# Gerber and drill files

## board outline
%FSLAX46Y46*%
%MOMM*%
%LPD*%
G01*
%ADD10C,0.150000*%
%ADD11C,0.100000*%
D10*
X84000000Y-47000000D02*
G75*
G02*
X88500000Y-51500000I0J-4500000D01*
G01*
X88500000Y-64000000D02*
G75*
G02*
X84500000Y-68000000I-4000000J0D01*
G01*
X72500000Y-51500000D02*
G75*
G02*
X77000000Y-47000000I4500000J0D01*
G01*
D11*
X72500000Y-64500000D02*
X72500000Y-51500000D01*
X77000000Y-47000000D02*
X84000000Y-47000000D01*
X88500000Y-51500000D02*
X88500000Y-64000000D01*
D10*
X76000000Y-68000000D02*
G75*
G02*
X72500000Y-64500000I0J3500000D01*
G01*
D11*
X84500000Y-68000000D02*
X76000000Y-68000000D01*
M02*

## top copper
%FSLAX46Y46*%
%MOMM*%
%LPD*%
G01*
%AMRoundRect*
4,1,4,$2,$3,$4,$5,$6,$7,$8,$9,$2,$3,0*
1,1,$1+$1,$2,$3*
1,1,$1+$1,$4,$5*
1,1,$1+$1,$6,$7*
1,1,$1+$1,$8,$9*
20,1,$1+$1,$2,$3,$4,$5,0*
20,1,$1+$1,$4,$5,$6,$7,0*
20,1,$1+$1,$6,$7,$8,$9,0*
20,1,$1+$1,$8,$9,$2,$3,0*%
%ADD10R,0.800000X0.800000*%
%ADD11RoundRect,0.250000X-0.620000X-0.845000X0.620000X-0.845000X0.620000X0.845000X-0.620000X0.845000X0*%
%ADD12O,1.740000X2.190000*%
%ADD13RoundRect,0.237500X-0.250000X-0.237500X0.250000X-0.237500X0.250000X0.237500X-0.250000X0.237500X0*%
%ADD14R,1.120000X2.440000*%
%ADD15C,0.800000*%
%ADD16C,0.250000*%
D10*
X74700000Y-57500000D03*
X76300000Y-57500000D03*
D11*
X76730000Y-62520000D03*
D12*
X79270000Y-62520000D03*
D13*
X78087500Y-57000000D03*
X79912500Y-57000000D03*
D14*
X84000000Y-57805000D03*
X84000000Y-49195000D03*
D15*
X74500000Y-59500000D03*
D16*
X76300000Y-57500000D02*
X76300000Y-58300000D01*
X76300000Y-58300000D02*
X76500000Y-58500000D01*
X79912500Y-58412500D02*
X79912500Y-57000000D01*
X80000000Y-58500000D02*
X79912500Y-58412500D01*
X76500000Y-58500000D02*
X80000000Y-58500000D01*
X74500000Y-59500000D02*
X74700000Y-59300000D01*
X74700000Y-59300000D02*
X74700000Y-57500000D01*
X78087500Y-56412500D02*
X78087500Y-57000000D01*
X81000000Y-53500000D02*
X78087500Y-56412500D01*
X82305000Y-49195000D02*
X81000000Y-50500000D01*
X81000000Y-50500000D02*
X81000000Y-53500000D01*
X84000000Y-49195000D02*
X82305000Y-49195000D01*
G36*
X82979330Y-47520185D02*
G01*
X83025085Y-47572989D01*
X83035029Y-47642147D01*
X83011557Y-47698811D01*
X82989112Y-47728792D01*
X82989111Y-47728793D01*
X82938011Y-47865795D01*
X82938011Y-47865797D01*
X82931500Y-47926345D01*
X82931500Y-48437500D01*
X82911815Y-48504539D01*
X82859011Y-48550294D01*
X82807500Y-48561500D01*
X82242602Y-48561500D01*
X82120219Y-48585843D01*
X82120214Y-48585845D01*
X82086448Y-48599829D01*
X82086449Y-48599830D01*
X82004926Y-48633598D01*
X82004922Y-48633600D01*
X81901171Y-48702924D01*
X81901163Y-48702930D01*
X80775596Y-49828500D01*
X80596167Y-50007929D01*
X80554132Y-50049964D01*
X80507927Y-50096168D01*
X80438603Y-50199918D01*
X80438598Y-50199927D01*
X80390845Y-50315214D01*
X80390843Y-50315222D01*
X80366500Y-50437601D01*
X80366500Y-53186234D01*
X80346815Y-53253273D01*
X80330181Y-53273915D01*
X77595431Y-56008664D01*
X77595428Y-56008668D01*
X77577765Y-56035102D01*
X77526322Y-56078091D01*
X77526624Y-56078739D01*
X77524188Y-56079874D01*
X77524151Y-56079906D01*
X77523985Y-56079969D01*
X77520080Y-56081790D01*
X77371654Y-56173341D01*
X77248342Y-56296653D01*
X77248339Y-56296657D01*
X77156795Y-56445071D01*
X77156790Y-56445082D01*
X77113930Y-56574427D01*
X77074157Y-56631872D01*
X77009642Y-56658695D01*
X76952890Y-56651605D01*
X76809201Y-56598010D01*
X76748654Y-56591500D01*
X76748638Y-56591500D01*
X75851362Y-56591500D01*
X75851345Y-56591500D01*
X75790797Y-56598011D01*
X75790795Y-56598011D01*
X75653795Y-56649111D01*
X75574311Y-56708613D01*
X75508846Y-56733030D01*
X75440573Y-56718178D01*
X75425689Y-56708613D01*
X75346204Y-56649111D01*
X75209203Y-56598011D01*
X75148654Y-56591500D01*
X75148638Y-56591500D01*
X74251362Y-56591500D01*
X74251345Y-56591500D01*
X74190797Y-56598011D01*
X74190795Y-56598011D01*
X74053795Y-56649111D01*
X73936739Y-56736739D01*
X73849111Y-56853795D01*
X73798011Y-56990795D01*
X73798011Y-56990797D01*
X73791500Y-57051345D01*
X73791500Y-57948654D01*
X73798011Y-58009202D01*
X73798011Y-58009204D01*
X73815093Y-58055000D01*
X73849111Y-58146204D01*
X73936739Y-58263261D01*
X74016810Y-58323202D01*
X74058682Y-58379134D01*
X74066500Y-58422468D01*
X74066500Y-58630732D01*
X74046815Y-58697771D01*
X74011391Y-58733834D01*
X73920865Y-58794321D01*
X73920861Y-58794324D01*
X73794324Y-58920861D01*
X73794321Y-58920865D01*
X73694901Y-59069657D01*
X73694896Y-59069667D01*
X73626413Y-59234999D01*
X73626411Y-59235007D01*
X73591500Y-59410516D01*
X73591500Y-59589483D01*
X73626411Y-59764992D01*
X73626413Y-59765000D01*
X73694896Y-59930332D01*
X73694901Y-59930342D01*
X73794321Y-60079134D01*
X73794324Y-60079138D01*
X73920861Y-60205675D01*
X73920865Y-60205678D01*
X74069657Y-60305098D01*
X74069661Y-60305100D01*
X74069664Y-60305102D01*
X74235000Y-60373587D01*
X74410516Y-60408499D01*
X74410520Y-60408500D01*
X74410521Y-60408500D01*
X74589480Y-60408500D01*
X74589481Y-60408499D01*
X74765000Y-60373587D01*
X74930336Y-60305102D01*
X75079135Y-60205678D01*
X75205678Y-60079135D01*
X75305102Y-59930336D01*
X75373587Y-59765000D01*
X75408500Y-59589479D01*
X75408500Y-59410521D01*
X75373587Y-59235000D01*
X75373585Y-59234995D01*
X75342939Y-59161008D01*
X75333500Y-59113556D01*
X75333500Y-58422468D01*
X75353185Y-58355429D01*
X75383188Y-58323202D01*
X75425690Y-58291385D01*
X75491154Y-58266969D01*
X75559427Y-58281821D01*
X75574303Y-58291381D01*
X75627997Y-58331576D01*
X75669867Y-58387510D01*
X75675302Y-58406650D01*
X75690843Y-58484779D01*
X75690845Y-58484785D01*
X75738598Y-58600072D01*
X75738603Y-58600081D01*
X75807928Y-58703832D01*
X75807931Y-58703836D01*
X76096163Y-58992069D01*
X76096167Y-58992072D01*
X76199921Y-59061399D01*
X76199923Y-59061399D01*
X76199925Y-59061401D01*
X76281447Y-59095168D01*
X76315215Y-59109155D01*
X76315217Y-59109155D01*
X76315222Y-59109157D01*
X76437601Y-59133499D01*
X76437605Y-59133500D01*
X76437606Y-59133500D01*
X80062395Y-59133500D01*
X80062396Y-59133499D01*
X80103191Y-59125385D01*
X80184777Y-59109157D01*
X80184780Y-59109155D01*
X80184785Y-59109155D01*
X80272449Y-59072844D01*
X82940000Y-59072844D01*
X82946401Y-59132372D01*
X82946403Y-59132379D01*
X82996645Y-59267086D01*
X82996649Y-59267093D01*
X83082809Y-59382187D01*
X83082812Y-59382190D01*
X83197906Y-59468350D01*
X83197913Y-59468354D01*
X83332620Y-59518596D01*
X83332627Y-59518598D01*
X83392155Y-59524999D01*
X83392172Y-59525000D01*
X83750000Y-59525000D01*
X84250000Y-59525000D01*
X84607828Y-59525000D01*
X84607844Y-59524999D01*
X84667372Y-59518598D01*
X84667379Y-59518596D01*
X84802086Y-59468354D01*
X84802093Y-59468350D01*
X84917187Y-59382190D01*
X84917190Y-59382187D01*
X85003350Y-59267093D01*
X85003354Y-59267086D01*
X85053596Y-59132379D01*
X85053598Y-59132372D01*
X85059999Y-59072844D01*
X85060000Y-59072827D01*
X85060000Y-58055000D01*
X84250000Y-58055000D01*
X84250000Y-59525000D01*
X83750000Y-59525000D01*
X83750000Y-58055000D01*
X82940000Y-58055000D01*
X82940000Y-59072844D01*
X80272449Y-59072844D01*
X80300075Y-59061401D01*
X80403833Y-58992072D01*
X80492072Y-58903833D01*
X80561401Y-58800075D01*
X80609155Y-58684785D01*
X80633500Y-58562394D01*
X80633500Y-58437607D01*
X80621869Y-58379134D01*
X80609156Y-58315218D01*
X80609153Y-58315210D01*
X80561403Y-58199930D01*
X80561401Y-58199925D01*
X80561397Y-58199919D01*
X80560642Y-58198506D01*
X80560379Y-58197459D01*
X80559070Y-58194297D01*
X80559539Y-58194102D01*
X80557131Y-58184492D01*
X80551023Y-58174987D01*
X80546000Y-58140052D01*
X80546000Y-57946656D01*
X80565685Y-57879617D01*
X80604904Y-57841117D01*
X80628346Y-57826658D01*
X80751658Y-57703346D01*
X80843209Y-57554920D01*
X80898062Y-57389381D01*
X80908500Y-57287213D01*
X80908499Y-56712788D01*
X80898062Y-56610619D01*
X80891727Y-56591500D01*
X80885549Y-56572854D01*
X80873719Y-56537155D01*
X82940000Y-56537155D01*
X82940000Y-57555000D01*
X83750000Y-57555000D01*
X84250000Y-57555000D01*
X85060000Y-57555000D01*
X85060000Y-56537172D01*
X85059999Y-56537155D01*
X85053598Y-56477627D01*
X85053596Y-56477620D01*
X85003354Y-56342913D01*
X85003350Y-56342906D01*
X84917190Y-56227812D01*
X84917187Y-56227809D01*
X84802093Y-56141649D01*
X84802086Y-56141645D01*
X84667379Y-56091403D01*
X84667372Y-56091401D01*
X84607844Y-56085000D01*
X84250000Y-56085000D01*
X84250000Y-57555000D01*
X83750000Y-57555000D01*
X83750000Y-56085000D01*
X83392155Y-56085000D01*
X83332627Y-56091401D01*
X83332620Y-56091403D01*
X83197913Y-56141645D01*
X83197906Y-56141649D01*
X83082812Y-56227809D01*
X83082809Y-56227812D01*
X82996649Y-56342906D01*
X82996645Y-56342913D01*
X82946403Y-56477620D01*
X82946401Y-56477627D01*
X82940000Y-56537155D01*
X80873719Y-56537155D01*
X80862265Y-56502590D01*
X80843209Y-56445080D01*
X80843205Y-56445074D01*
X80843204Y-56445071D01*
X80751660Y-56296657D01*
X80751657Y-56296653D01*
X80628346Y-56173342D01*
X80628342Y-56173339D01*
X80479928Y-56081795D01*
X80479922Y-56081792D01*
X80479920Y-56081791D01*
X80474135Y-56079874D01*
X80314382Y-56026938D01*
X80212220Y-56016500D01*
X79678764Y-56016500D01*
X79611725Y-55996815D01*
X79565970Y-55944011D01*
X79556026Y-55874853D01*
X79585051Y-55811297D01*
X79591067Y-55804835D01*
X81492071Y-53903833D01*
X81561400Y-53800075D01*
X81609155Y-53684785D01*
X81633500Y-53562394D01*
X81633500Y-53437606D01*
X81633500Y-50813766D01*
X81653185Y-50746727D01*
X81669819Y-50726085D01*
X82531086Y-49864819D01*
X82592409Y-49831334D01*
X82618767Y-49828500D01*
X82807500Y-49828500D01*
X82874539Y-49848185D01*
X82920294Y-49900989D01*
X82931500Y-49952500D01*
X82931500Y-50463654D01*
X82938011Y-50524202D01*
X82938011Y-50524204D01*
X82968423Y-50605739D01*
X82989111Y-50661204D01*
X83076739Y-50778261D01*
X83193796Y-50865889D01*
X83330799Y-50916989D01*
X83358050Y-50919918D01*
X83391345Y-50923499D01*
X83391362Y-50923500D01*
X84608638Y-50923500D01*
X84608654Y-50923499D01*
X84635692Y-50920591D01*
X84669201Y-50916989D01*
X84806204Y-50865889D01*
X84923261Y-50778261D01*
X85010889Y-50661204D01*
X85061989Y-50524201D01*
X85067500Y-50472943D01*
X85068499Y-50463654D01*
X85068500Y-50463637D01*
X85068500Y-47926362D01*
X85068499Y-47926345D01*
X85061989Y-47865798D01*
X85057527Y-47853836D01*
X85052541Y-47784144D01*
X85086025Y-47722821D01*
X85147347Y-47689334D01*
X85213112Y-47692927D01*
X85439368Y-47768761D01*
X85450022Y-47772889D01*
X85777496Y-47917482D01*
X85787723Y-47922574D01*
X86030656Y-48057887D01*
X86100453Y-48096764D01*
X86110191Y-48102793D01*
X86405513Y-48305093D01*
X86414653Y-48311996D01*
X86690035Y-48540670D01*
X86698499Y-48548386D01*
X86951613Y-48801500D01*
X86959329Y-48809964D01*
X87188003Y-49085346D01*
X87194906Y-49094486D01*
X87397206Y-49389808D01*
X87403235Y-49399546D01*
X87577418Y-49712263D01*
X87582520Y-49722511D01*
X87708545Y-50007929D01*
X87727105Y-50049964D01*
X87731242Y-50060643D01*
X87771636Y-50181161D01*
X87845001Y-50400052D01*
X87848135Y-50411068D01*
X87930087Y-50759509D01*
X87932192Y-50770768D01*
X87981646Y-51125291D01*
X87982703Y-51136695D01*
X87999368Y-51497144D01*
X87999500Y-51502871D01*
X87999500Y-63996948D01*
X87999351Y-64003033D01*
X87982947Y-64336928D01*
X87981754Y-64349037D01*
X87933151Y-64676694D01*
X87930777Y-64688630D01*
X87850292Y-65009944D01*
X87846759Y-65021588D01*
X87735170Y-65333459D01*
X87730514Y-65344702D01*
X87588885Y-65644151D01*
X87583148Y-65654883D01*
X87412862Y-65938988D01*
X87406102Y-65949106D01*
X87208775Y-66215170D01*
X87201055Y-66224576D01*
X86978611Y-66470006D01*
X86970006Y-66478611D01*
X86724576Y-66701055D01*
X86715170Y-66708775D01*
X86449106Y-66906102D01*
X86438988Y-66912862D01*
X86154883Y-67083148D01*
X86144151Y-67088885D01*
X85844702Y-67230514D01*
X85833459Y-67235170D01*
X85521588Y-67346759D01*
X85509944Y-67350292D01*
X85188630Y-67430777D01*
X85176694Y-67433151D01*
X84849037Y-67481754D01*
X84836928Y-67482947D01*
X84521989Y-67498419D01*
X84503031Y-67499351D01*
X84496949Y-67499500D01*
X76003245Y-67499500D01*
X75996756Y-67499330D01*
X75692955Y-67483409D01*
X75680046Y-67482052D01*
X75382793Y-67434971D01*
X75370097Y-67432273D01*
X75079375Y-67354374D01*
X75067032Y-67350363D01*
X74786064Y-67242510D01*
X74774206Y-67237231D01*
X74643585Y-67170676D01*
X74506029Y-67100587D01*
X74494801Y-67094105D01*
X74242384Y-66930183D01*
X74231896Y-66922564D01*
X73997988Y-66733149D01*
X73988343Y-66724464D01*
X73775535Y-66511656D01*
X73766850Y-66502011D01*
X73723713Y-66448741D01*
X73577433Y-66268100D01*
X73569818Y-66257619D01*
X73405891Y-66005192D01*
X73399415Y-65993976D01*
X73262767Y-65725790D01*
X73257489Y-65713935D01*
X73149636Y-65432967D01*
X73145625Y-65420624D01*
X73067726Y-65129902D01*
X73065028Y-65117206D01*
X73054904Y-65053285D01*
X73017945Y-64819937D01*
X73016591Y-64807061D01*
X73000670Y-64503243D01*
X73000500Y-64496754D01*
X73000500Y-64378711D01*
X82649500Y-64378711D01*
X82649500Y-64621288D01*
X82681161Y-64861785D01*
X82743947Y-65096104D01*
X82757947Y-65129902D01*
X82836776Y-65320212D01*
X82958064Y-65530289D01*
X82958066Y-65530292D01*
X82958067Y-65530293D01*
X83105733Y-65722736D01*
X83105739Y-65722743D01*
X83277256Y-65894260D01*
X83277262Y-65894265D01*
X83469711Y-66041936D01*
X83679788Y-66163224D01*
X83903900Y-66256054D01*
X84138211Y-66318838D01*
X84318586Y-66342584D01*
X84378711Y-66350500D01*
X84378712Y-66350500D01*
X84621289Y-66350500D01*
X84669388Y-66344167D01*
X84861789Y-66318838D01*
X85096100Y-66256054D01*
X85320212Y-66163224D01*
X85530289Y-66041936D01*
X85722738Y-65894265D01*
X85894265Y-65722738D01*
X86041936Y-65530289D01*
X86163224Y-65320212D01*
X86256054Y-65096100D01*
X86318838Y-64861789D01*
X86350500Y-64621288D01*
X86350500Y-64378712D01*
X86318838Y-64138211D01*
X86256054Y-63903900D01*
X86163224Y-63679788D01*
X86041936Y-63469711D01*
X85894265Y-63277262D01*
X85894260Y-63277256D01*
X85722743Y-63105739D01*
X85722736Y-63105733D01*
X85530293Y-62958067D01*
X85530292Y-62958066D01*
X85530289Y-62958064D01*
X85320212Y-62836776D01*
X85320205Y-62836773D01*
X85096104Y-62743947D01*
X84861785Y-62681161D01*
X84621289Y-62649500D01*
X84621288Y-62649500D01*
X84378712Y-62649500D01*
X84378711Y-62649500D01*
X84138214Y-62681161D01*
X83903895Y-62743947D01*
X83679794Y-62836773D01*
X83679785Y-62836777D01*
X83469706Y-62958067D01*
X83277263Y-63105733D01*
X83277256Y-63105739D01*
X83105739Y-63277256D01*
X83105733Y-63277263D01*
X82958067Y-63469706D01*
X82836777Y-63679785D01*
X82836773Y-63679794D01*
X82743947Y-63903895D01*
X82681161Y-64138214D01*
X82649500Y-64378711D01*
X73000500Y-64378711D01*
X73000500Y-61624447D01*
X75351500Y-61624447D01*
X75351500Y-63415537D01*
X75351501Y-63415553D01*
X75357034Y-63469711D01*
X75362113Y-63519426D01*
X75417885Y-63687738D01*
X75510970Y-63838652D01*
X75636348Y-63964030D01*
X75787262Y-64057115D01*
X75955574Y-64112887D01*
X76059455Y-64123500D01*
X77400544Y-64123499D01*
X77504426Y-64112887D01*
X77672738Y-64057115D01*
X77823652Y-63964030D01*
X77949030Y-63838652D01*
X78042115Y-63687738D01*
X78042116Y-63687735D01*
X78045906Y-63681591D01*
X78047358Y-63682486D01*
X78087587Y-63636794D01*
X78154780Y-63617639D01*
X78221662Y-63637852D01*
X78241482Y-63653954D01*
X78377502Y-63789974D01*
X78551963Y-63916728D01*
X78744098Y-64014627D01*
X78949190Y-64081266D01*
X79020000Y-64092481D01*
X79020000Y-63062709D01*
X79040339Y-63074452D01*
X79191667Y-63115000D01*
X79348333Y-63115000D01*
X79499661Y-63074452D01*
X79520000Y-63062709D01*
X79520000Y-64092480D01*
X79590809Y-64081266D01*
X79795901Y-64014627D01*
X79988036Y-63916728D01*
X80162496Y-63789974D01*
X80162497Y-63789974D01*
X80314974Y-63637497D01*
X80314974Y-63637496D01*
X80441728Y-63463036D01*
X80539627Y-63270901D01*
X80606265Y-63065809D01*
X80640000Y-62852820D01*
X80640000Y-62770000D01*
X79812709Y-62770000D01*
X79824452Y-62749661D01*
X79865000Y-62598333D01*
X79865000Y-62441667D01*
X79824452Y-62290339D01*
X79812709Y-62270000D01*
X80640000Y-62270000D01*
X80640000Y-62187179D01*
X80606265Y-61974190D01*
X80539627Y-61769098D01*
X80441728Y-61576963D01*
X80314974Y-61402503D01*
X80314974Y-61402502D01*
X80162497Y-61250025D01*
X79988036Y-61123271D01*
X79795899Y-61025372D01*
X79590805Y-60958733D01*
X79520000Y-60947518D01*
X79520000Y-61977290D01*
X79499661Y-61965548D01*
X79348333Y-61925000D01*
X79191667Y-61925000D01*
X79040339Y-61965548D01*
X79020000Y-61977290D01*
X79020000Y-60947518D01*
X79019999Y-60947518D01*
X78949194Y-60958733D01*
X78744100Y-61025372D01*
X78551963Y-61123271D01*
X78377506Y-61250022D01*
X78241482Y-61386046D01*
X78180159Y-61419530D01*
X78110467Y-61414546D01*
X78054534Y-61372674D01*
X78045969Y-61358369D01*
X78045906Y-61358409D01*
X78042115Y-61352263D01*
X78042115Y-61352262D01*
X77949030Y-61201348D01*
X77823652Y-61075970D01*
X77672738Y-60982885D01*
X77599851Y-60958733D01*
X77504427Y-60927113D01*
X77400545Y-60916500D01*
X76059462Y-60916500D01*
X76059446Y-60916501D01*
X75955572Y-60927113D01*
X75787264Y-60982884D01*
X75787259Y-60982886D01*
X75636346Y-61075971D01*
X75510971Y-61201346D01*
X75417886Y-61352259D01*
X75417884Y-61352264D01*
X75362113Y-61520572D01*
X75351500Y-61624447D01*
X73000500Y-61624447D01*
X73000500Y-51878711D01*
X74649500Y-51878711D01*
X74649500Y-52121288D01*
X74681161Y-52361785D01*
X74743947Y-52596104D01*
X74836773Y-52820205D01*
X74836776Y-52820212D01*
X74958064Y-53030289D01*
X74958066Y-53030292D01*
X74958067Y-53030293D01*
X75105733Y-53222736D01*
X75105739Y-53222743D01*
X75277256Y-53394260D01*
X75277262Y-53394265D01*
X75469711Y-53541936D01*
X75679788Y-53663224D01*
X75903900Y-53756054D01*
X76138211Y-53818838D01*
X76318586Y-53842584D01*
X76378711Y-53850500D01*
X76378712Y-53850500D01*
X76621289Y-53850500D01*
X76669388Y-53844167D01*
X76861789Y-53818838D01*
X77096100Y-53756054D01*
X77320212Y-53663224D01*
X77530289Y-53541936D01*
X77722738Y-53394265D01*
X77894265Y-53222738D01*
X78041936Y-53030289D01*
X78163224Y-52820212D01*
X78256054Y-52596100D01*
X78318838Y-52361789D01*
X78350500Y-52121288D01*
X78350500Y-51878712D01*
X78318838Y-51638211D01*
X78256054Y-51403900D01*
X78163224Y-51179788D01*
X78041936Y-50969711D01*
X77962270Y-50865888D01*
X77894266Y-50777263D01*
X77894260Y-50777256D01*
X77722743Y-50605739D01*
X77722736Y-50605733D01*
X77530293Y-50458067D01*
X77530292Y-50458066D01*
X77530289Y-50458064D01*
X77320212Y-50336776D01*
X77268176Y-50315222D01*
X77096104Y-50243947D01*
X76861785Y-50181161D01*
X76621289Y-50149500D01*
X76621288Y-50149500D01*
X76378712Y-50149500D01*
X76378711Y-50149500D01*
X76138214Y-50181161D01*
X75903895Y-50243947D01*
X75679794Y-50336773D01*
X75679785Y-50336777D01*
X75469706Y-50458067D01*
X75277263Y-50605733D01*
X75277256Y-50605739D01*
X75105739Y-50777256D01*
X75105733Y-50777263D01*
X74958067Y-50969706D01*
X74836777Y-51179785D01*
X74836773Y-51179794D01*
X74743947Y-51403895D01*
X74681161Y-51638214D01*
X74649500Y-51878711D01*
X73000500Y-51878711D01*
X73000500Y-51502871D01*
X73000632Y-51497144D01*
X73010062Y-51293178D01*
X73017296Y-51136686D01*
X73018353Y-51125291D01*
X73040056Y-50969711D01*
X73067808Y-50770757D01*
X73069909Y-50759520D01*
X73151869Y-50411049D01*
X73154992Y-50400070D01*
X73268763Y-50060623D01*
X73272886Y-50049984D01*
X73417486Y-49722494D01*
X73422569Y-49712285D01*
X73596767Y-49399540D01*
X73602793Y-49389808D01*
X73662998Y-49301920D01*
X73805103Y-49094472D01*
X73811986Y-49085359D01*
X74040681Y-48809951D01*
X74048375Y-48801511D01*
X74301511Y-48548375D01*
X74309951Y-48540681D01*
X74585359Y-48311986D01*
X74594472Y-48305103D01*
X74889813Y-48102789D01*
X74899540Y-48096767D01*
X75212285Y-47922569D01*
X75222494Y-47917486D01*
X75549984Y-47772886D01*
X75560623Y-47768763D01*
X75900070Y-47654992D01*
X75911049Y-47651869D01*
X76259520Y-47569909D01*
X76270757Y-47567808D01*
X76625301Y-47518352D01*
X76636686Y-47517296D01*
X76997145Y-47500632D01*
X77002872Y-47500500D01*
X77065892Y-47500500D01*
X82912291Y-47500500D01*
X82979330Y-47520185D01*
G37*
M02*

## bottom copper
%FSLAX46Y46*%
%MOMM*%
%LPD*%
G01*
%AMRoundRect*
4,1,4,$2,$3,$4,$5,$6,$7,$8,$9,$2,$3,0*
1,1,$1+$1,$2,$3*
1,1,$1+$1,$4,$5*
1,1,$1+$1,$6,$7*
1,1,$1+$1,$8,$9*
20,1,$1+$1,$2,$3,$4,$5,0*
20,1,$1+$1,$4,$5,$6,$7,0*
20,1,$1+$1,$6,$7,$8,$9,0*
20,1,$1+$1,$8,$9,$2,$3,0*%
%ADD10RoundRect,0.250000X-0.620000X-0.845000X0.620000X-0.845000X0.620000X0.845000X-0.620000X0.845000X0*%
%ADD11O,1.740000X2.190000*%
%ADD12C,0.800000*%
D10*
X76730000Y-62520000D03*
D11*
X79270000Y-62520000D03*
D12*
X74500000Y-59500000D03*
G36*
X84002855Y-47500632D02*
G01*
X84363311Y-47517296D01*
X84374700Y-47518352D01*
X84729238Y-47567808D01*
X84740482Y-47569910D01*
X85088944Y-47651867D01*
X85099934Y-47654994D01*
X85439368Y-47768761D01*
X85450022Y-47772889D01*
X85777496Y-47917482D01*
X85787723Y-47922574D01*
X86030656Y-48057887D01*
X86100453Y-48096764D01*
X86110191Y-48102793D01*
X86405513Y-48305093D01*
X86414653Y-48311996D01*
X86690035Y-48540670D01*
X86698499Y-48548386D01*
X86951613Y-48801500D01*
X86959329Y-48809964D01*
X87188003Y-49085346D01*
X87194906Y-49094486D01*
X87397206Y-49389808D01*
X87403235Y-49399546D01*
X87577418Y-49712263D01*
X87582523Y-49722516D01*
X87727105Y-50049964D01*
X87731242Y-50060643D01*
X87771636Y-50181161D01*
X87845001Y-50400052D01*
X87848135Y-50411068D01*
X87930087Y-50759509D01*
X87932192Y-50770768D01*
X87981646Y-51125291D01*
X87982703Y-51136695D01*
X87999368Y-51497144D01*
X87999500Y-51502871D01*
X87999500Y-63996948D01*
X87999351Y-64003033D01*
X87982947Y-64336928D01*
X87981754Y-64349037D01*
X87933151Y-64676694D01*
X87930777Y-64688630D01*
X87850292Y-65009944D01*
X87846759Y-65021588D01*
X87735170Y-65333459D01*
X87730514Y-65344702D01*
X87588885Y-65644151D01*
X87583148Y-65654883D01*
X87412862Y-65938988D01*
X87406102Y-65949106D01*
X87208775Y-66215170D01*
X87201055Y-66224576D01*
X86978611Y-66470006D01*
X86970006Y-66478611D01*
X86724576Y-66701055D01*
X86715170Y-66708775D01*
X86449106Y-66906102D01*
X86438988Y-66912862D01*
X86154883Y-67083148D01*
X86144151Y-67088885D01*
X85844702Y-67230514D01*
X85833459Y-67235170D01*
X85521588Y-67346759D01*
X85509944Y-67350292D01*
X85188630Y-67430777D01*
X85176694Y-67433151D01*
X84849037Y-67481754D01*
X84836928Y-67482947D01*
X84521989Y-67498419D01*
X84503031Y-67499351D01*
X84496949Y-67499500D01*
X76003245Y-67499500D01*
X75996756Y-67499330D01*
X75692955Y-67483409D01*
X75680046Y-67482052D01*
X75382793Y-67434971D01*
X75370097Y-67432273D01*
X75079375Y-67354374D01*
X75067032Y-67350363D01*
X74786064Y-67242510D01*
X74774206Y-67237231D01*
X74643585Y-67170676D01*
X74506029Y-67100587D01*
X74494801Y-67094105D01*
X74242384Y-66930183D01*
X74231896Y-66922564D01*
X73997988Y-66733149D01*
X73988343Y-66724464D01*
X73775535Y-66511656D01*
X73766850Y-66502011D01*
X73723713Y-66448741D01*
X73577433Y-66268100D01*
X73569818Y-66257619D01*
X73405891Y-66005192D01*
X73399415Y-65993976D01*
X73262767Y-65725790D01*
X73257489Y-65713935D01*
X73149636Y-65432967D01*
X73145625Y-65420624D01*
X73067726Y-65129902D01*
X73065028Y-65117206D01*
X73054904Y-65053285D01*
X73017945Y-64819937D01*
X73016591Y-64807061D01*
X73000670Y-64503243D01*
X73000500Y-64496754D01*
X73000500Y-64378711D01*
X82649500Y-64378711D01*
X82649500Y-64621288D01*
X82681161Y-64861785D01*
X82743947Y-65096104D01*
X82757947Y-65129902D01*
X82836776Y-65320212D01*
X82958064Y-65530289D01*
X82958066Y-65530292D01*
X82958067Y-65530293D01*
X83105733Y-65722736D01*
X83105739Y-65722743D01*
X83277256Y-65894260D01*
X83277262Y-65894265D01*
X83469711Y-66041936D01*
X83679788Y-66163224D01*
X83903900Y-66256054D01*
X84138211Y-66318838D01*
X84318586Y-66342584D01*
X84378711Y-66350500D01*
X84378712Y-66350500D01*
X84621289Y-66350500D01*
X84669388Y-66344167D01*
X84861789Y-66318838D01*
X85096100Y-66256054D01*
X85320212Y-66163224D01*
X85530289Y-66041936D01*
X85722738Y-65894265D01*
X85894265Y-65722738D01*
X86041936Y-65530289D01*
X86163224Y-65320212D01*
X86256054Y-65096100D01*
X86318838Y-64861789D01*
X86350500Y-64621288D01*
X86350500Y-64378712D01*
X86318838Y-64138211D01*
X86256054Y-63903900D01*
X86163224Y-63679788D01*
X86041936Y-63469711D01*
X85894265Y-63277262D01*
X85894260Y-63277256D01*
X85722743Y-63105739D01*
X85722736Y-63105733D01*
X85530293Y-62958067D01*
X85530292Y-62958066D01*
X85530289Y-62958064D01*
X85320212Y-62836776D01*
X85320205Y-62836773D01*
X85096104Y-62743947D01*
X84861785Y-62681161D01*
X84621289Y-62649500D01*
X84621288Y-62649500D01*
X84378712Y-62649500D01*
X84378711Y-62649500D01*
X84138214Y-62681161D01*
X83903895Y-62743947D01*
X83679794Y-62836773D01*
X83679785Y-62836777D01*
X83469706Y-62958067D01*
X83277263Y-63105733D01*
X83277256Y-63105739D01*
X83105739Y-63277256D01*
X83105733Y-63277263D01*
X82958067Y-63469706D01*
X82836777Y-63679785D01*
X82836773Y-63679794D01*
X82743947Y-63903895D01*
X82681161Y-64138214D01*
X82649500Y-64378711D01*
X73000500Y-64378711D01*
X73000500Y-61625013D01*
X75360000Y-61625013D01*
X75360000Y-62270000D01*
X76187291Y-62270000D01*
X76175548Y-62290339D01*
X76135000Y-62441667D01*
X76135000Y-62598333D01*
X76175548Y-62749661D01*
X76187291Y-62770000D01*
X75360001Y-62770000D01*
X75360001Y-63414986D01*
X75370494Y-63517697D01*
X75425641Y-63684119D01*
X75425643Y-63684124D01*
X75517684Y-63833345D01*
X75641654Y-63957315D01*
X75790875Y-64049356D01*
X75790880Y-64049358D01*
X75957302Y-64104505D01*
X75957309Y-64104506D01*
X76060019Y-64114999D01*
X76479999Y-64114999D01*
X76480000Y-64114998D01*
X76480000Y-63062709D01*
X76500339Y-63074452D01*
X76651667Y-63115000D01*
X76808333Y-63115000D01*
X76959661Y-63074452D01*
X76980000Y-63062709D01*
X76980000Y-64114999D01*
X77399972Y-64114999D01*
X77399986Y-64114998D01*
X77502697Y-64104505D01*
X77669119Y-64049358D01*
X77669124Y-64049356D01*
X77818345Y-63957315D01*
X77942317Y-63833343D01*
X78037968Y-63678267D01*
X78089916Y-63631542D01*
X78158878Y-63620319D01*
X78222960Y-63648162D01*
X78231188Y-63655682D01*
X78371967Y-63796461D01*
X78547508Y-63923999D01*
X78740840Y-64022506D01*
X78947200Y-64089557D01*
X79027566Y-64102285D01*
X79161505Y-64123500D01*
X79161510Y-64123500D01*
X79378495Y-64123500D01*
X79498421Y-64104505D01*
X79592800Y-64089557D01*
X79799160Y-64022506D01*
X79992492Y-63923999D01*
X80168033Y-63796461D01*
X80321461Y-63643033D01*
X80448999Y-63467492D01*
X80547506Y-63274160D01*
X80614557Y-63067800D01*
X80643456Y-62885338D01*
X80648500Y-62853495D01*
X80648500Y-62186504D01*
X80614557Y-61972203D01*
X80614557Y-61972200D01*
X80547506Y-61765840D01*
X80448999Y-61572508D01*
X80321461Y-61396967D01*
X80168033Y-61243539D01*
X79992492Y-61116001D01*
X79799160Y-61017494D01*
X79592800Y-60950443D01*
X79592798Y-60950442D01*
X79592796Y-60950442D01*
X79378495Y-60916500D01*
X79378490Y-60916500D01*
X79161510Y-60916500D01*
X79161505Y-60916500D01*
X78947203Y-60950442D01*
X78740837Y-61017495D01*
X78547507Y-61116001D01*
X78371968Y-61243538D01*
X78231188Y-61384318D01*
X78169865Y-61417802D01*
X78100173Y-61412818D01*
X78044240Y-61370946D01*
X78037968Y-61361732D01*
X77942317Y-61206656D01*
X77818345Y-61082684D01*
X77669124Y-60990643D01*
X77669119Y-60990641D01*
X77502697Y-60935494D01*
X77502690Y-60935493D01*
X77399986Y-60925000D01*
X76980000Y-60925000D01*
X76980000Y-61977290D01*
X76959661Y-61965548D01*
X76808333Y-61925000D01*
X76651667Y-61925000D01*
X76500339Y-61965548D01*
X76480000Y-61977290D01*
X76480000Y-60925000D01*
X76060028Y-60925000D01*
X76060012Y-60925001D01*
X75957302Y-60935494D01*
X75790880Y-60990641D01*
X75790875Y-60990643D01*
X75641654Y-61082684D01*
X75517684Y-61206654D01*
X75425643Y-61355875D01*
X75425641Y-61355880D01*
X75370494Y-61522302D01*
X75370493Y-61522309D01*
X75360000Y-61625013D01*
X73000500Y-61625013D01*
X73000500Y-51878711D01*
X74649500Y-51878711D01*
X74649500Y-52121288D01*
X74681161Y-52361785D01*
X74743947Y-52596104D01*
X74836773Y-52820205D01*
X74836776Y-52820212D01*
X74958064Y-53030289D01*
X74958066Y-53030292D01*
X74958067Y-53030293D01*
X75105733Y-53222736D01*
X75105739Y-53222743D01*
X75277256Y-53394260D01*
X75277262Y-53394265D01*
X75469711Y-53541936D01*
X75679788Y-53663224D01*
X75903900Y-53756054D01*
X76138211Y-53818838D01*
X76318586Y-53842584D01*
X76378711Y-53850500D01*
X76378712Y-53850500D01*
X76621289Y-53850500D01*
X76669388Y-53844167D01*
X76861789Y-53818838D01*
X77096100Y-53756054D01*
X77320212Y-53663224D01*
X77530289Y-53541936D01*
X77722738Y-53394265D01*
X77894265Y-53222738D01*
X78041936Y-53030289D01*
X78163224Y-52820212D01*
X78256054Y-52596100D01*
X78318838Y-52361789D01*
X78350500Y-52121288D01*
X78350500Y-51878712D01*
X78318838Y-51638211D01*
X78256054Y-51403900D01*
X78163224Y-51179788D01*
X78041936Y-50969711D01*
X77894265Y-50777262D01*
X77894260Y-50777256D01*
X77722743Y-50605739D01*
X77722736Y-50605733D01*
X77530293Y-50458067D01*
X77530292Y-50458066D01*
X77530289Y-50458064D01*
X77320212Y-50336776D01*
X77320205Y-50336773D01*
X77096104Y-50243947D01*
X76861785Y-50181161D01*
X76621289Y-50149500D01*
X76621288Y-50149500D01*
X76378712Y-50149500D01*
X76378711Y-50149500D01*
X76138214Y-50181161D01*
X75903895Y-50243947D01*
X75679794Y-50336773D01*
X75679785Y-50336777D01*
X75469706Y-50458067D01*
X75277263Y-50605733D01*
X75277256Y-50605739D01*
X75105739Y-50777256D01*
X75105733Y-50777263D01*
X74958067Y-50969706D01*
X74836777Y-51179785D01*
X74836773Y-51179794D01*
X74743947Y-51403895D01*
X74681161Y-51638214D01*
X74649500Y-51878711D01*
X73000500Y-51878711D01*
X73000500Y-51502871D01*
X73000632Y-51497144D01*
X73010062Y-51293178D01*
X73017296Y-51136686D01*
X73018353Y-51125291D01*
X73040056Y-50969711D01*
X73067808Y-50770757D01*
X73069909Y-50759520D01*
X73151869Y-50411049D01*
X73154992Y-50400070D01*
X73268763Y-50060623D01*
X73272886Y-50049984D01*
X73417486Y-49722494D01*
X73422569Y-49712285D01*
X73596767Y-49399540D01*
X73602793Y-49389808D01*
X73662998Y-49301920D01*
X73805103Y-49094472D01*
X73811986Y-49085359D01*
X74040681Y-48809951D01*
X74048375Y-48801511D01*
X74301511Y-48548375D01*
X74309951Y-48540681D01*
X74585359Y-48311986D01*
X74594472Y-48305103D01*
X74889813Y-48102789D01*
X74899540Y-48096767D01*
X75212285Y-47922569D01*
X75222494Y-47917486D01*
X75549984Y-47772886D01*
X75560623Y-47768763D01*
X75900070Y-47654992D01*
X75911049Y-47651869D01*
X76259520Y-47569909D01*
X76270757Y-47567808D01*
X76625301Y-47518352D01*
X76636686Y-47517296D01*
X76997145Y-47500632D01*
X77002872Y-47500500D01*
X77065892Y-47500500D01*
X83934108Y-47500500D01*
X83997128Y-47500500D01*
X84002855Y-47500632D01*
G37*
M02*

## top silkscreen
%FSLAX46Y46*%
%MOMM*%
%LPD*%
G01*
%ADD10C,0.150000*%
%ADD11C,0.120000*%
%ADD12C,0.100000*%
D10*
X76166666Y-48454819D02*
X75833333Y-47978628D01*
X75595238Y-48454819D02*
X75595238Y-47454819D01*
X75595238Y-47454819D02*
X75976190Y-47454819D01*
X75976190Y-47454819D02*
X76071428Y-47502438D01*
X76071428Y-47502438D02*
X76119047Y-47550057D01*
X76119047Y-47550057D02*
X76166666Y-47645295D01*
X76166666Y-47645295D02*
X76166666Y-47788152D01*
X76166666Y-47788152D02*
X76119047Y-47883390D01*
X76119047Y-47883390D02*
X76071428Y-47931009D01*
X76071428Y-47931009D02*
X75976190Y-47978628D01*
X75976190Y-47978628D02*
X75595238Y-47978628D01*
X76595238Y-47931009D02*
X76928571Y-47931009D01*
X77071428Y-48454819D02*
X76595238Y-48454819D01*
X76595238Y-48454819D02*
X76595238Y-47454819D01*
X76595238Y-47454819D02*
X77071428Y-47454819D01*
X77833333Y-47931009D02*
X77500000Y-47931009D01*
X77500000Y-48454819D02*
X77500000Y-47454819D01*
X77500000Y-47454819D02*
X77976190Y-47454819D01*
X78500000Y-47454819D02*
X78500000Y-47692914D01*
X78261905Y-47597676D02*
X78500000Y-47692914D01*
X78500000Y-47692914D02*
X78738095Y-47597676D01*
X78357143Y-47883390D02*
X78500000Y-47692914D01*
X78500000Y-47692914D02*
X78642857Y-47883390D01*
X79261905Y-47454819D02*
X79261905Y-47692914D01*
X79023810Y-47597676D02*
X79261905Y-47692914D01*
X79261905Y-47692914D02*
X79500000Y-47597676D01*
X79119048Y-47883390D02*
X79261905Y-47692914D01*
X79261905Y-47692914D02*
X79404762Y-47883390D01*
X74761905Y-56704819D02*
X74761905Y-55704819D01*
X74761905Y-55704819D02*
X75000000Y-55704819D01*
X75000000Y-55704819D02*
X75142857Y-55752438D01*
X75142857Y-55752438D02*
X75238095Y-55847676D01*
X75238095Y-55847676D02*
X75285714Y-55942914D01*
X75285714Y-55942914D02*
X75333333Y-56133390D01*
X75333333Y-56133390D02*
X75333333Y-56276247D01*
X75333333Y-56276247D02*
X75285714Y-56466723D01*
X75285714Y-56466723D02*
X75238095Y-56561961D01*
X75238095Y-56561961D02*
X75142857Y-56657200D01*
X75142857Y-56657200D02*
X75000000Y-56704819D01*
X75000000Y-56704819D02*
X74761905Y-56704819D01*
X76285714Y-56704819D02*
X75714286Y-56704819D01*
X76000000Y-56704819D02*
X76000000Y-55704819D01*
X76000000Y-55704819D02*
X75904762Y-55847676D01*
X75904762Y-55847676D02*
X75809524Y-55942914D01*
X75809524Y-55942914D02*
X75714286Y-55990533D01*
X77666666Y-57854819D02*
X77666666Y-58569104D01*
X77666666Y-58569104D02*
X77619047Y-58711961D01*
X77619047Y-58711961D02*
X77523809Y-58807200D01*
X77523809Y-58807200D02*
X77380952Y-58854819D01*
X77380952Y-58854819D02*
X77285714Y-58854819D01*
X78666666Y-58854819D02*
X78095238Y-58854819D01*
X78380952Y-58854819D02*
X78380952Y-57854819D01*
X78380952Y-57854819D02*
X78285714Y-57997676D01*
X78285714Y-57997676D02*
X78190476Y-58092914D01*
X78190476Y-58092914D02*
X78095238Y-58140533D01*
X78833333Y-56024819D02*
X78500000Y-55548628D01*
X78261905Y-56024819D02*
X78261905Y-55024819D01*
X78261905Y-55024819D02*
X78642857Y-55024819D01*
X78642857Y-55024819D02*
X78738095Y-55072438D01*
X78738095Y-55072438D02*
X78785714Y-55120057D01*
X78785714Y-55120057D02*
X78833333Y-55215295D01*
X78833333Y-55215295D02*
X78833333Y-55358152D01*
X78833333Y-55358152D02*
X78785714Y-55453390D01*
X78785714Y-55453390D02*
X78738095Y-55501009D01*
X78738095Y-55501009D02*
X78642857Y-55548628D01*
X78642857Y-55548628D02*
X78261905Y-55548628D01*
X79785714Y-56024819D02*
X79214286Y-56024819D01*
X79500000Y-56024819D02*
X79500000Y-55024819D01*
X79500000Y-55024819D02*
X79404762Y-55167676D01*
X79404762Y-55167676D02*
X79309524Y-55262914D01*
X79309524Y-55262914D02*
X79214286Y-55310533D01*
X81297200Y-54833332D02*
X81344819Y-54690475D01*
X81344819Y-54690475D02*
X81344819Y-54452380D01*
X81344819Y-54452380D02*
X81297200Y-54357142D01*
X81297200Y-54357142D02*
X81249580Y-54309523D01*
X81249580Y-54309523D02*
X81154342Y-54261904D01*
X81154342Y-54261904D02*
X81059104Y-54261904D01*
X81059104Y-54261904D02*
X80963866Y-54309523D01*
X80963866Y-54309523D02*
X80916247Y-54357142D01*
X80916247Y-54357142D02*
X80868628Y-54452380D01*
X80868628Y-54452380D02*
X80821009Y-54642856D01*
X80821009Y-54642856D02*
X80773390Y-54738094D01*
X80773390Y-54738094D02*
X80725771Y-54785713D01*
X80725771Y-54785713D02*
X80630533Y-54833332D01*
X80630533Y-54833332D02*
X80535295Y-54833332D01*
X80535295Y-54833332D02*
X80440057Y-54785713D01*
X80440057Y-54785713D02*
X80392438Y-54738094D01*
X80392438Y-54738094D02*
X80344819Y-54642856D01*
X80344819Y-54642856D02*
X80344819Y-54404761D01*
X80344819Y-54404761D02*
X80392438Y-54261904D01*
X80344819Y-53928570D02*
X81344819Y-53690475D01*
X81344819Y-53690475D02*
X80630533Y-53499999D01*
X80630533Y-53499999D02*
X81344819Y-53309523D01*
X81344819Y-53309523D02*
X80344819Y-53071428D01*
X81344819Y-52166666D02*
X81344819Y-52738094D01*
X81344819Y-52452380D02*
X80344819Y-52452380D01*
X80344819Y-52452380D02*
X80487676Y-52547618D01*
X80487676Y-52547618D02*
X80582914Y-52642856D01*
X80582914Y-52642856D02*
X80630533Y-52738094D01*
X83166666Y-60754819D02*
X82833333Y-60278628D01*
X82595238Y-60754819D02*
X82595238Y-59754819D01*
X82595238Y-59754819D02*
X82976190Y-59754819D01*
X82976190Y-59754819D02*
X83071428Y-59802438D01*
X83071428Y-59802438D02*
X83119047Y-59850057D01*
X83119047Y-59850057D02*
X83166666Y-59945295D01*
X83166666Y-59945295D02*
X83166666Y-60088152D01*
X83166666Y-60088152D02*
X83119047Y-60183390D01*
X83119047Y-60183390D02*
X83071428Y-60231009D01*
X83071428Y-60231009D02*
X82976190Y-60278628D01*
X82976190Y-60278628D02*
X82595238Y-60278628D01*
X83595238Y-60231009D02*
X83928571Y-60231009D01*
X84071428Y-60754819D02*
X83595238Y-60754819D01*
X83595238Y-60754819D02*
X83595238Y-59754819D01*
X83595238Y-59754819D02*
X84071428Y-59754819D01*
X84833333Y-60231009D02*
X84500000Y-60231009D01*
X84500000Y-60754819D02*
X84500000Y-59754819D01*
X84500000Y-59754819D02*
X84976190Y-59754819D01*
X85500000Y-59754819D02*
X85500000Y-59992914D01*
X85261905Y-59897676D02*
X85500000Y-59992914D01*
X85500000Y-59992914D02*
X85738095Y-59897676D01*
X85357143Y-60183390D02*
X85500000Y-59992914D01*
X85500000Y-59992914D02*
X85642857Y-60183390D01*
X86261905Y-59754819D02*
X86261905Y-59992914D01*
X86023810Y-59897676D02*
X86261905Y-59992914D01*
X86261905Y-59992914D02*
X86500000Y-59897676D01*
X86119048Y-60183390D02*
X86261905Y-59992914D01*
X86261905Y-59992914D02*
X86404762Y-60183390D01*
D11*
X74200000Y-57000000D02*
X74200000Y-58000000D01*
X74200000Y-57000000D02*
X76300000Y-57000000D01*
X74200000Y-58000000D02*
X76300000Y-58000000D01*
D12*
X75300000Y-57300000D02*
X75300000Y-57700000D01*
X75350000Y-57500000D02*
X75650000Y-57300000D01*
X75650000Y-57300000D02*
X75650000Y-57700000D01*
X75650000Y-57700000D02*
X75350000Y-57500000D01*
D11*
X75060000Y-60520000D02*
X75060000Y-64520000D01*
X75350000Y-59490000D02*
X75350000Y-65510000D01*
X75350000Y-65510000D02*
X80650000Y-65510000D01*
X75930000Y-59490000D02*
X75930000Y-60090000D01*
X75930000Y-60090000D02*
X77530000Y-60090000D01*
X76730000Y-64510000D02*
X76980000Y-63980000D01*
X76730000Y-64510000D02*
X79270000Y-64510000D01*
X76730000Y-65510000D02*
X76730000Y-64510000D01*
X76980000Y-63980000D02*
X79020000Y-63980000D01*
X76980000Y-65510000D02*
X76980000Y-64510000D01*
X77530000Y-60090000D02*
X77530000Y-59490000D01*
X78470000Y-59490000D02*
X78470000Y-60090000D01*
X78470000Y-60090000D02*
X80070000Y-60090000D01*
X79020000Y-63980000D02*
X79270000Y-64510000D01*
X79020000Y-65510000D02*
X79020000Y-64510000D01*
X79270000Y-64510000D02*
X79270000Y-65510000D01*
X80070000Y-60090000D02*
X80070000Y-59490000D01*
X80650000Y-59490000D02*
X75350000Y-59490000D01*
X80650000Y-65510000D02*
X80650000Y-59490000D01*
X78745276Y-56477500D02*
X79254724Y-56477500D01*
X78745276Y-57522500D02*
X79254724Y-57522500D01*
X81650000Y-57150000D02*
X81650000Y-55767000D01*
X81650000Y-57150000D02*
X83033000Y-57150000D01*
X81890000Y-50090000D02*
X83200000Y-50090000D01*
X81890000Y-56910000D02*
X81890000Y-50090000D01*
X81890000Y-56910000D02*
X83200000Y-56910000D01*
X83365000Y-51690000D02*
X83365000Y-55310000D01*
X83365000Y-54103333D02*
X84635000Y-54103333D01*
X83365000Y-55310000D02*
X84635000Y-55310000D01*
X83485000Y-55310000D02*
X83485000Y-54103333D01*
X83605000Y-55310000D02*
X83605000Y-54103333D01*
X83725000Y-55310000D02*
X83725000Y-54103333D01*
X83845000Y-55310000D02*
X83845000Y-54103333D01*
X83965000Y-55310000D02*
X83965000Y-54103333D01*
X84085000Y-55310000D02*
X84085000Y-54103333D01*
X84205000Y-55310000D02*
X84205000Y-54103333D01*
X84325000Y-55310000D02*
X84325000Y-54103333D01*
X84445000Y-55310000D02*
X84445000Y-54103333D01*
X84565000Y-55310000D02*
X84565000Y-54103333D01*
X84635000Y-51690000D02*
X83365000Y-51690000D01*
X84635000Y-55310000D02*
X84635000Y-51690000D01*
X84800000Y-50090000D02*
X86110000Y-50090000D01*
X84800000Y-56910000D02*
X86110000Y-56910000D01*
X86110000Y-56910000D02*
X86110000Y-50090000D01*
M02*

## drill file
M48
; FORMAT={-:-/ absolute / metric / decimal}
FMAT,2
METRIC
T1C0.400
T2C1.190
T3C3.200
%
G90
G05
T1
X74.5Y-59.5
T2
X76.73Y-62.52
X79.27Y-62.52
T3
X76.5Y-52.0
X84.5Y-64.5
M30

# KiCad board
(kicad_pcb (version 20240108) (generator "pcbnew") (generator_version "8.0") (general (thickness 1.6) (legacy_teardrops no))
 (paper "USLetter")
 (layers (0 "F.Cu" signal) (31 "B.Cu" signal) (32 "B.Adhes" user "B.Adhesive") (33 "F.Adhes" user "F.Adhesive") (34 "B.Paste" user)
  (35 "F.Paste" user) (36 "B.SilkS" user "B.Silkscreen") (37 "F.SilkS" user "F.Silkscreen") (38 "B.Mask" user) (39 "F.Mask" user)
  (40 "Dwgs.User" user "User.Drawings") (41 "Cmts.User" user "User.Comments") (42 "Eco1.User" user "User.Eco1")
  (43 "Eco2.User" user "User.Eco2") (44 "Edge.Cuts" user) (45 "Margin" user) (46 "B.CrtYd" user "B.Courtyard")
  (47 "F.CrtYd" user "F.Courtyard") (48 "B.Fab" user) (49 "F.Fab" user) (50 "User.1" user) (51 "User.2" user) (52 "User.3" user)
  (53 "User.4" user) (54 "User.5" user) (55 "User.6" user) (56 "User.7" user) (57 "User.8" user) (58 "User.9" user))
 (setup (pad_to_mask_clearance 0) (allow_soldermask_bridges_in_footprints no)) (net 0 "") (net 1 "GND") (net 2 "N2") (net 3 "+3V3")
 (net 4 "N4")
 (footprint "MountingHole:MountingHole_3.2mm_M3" (layer "F.Cu") (at 76.5 52)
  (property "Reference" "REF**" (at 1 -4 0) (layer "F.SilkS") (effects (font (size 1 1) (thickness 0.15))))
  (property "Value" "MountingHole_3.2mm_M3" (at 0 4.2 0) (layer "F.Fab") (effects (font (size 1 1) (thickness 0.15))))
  (pad "" np_thru_hole circle (at 0 0) (size 3.2 3.2) (drill 3.2) (layers "*.Cu" "*.Mask")))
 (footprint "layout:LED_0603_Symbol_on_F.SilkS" (layer "F.Cu") (at 75.5 57.5)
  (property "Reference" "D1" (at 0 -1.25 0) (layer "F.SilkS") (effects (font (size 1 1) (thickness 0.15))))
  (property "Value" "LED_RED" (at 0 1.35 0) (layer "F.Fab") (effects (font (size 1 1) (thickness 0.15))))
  (fp_line (start -1.3 -0.5) (end -1.3 0.5) (stroke (width 0.12) (type solid)) (layer "F.SilkS"))
  (fp_line (start -1.3 -0.5) (end 0.8 -0.5) (stroke (width 0.12) (type solid)) (layer "F.SilkS"))
  (fp_line (start -1.3 0.5) (end 0.8 0.5) (stroke (width 0.12) (type solid)) (layer "F.SilkS"))
  (fp_line (start -0.2 -0.2) (end -0.2 0.2) (stroke (width 0.1) (type solid)) (layer "F.SilkS"))
  (fp_line (start -0.15 0) (end 0.15 -0.2) (stroke (width 0.1) (type solid)) (layer "F.SilkS"))
  (fp_line (start 0.15 -0.2) (end 0.15 0.2) (stroke (width 0.1) (type solid)) (layer "F.SilkS"))
  (fp_line (start 0.15 0.2) (end -0.15 0) (stroke (width 0.1) (type solid)) (layer "F.SilkS"))
  (pad "1" smd rect (at -0.8 0 180) (size 0.8 0.8) (layers "F.Cu" "F.Paste" "F.Mask") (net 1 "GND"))
  (pad "2" smd rect (at 0.8 0 180) (size 0.8 0.8) (layers "F.Cu" "F.Paste" "F.Mask") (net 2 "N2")))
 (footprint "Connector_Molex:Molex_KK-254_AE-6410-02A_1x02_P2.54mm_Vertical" (layer "F.Cu") (at 76.73 62.52)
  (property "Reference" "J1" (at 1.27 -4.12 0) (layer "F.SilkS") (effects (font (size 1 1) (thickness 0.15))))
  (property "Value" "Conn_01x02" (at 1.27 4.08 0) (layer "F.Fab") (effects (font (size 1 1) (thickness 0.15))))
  (fp_line (start -1.67 -2) (end -1.67 2) (stroke (width 0.12) (type solid)) (layer "F.SilkS"))
  (fp_line (start -1.38 -3.03) (end -1.38 2.99) (stroke (width 0.12) (type solid)) (layer "F.SilkS"))
  (fp_line (start -1.38 2.99) (end 3.92 2.99) (stroke (width 0.12) (type solid)) (layer "F.SilkS"))
  (fp_line (start -0.8 -3.03) (end -0.8 -2.43) (stroke (width 0.12) (type solid)) (layer "F.SilkS"))
  (fp_line (start -0.8 -2.43) (end 0.8 -2.43) (stroke (width 0.12) (type solid)) (layer "F.SilkS"))
  (fp_line (start 0 1.99) (end 0.25 1.46) (stroke (width 0.12) (type solid)) (layer "F.SilkS"))
  (fp_line (start 0 1.99) (end 2.54 1.99) (stroke (width 0.12) (type solid)) (layer "F.SilkS"))
  (fp_line (start 0 2.99) (end 0 1.99) (stroke (width 0.12) (type solid)) (layer "F.SilkS"))
  (fp_line (start 0.25 1.46) (end 2.29 1.46) (stroke (width 0.12) (type solid)) (layer "F.SilkS"))
  (fp_line (start 0.25 2.99) (end 0.25 1.99) (stroke (width 0.12) (type solid)) (layer "F.SilkS"))
  (fp_line (start 0.8 -2.43) (end 0.8 -3.03) (stroke (width 0.12) (type solid)) (layer "F.SilkS"))
  (fp_line (start 1.74 -3.03) (end 1.74 -2.43) (stroke (width 0.12) (type solid)) (layer "F.SilkS"))
  (fp_line (start 1.74 -2.43) (end 3.34 -2.43) (stroke (width 0.12) (type solid)) (layer "F.SilkS"))
  (fp_line (start 2.29 1.46) (end 2.54 1.99) (stroke (width 0.12) (type solid)) (layer "F.SilkS"))
  (fp_line (start 2.29 2.99) (end 2.29 1.99) (stroke (width 0.12) (type solid)) (layer "F.SilkS"))
  (fp_line (start 2.54 1.99) (end 2.54 2.99) (stroke (width 0.12) (type solid)) (layer "F.SilkS"))
  (fp_line (start 3.34 -2.43) (end 3.34 -3.03) (stroke (width 0.12) (type solid)) (layer "F.SilkS"))
  (fp_line (start 3.92 -3.03) (end -1.38 -3.03) (stroke (width 0.12) (type solid)) (layer "F.SilkS"))
  (fp_line (start 3.92 2.99) (end 3.92 -3.03) (stroke (width 0.12) (type solid)) (layer "F.SilkS"))
  (pad "1" thru_hole roundrect (at 0 0) (size 1.74 2.19) (drill 1.19) (layers "*.Cu" "*.Mask") (remove_unused_layers no)
   (roundrect_rratio 0.143678) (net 1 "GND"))
  (pad "2" thru_hole oval (at 2.54 0) (size 1.74 2.19) (drill 1.19) (layers "*.Cu" "*.Mask") (remove_unused_layers no) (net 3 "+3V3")))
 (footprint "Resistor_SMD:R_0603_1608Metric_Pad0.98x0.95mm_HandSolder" (layer "F.Cu") (at 79 57)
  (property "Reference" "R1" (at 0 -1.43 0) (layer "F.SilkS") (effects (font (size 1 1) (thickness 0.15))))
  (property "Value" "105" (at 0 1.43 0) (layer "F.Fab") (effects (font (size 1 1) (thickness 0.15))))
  (fp_line (start -0.254724 -0.5225) (end 0.254724 -0.5225) (stroke (width 0.12) (type solid)) (layer "F.SilkS"))
  (fp_line (start -0.254724 0.5225) (end 0.254724 0.5225) (stroke (width 0.12) (type solid)) (layer "F.SilkS"))
  (pad "1" smd roundrect (at -0.9125 0) (size 0.975 0.95) (layers "F.Cu" "F.Paste" "F.Mask") (roundrect_rratio 0.25) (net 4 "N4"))
  (pad "2" smd roundrect (at 0.9125 0) (size 0.975 0.95) (layers "F.Cu" "F.Paste" "F.Mask") (roundrect_rratio 0.25) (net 2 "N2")))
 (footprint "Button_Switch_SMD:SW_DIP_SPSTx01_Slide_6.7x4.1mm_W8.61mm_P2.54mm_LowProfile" (layer "F.Cu") (at 84 53.5 90)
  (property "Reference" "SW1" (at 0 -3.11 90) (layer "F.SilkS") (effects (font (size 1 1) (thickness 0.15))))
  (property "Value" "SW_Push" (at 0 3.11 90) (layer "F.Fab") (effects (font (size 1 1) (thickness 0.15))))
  (fp_line (start -3.65 -2.35) (end -2.267 -2.35) (stroke (width 0.12) (type solid)) (layer "F.SilkS"))
  (fp_line (start -3.65 -2.35) (end -3.65 -0.967) (stroke (width 0.12) (type solid)) (layer "F.SilkS"))
  (fp_line (start 3.41 -2.11) (end 3.41 -0.8) (stroke (width 0.12) (type solid)) (layer "F.SilkS"))
  (fp_line (start -3.41 -2.11) (end 3.41 -2.11) (stroke (width 0.12) (type solid)) (layer "F.SilkS"))
  (fp_line (start -3.41 -2.11) (end -3.41 -0.8) (stroke (width 0.12) (type solid)) (layer "F.SilkS"))
  (fp_line (start 1.81 -0.635) (end -1.81 -0.635) (stroke (width 0.12) (type solid)) (layer "F.SilkS"))
  (fp_line (start -0.603333 -0.635) (end -0.603333 0.635) (stroke (width 0.12) (type solid)) (layer "F.SilkS"))
  (fp_line (start -1.81 -0.635) (end -1.81 0.635) (stroke (width 0.12) (type solid)) (layer "F.SilkS"))
  (fp_line (start -1.81 -0.515) (end -0.603333 -0.515) (stroke (width 0.12) (type solid)) (layer "F.SilkS"))
  (fp_line (start -1.81 -0.395) (end -0.603333 -0.395) (stroke (width 0.12) (type solid)) (layer "F.SilkS"))
  (fp_line (start -1.81 -0.275) (end -0.603333 -0.275) (stroke (width 0.12) (type solid)) (layer "F.SilkS"))
  (fp_line (start -1.81 -0.155) (end -0.603333 -0.155) (stroke (width 0.12) (type solid)) (layer "F.SilkS"))
  (fp_line (start -1.81 -0.035) (end -0.603333 -0.035) (stroke (width 0.12) (type solid)) (layer "F.SilkS"))
  (fp_line (start -1.81 0.085) (end -0.603333 0.085) (stroke (width 0.12) (type solid)) (layer "F.SilkS"))
  (fp_line (start -1.81 0.205) (end -0.603333 0.205) (stroke (width 0.12) (type solid)) (layer "F.SilkS"))
  (fp_line (start -1.81 0.325) (end -0.603333 0.325) (stroke (width 0.12) (type solid)) (layer "F.SilkS"))
  (fp_line (start -1.81 0.445) (end -0.603333 0.445) (stroke (width 0.12) (type solid)) (layer "F.SilkS"))
  (fp_line (start -1.81 0.565) (end -0.603333 0.565) (stroke (width 0.12) (type solid)) (layer "F.SilkS"))
  (fp_line (start 1.81 0.635) (end 1.81 -0.635) (stroke (width 0.12) (type solid)) (layer "F.SilkS"))
  (fp_line (start -1.81 0.635) (end 1.81 0.635) (stroke (width 0.12) (type solid)) (layer "F.SilkS"))
  (fp_line (start 3.41 0.8) (end 3.41 2.11) (stroke (width 0.12) (type solid)) (layer "F.SilkS"))
  (fp_line (start -3.41 0.8) (end -3.41 2.11) (stroke (width 0.12) (type solid)) (layer "F.SilkS"))
  (fp_line (start -3.41 2.11) (end 3.41 2.11) (stroke (width 0.12) (type solid)) (layer "F.SilkS"))
  (pad "1" smd rect (at -4.305 0 90) (size 2.44 1.12) (layers "F.Cu" "F.Paste" "F.Mask") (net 3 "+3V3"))
  (pad "2" smd rect (at 4.305 0 90) (size 2.44 1.12) (layers "F.Cu" "F.Paste" "F.Mask") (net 4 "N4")))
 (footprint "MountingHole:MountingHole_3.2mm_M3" (layer "F.Cu") (at 84.5 64.5)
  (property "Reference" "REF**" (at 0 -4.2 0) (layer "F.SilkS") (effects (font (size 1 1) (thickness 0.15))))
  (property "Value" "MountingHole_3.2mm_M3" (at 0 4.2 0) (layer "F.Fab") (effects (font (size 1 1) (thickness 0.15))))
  (pad "" np_thru_hole circle (at 0 0) (size 3.2 3.2) (drill 3.2) (layers "*.Cu" "*.Mask")))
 (gr_arc (start 84 47) (mid 87.181981 48.318019) (end 88.5 51.5) (stroke (width 0.15) (type default)) (layer "Edge.Cuts"))
 (gr_arc (start 88.5 64) (mid 87.328427 66.828427) (end 84.5 68) (stroke (width 0.15) (type default)) (layer "Edge.Cuts"))
 (gr_arc (start 72.5 51.5) (mid 73.818019 48.318019) (end 77 47) (stroke (width 0.15) (type default)) (layer "Edge.Cuts"))
 (gr_line (start 72.5 64.5) (end 72.5 51.5) (stroke (width 0.1) (type default)) (layer "Edge.Cuts"))
 (gr_line (start 77 47) (end 84 47) (stroke (width 0.1) (type default)) (layer "Edge.Cuts"))
 (gr_line (start 88.5 51.5) (end 88.5 64) (stroke (width 0.1) (type default)) (layer "Edge.Cuts"))
 (gr_arc (start 76 68) (mid 73.525126 66.974874) (end 72.5 64.5) (stroke (width 0.15) (type default)) (layer "Edge.Cuts"))
 (gr_line (start 84.5 68) (end 76 68) (stroke (width 0.1) (type default)) (layer "Edge.Cuts"))
 (segment (start 76.3 57.5) (end 76.3 58.3) (width 0.25) (layer "F.Cu") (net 2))
 (segment (start 76.3 58.3) (end 76.5 58.5) (width 0.25) (layer "F.Cu") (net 2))
 (segment (start 79.9125 58.4125) (end 79.9125 57) (width 0.25) (layer "F.Cu") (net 2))
 (segment (start 80 58.5) (end 79.9125 58.4125) (width 0.25) (layer "F.Cu") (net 2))
 (segment (start 76.5 58.5) (end 80 58.5) (width 0.25) (layer "F.Cu") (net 2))
 (segment (start 74.5 59.5) (end 74.7 59.3) (width 0.25) (layer "F.Cu") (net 1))
 (segment (start 74.7 59.3) (end 74.7 57.5) (width 0.25) (layer "F.Cu") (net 1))
 (via (at 74.5 59.5) (size 0.8) (drill 0.4) (layers "F.Cu" "B.Cu") (free yes) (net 1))
 (segment (start 78.0875 56.4125) (end 78.0875 57) (width 0.25) (layer "F.Cu") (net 4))
 (segment (start 81 53.5) (end 78.0875 56.4125) (width 0.25) (layer "F.Cu") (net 4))
 (segment (start 82.305 49.195) (end 81 50.5) (width 0.25) (layer "F.Cu") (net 4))
 (segment (start 81 50.5) (end 81 53.5) (width 0.25) (layer "F.Cu") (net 4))
 (segment (start 84 49.195) (end 82.305 49.195) (width 0.25) (layer "F.Cu") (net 4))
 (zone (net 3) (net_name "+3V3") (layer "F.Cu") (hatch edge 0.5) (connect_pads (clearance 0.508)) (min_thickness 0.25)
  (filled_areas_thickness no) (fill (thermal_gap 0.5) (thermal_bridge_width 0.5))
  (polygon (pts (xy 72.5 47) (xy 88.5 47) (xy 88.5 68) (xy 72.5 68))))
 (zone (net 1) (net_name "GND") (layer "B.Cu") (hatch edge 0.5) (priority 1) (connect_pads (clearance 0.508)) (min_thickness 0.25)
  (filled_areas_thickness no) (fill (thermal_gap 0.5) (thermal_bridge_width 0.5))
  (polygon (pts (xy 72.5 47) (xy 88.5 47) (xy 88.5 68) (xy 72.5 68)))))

